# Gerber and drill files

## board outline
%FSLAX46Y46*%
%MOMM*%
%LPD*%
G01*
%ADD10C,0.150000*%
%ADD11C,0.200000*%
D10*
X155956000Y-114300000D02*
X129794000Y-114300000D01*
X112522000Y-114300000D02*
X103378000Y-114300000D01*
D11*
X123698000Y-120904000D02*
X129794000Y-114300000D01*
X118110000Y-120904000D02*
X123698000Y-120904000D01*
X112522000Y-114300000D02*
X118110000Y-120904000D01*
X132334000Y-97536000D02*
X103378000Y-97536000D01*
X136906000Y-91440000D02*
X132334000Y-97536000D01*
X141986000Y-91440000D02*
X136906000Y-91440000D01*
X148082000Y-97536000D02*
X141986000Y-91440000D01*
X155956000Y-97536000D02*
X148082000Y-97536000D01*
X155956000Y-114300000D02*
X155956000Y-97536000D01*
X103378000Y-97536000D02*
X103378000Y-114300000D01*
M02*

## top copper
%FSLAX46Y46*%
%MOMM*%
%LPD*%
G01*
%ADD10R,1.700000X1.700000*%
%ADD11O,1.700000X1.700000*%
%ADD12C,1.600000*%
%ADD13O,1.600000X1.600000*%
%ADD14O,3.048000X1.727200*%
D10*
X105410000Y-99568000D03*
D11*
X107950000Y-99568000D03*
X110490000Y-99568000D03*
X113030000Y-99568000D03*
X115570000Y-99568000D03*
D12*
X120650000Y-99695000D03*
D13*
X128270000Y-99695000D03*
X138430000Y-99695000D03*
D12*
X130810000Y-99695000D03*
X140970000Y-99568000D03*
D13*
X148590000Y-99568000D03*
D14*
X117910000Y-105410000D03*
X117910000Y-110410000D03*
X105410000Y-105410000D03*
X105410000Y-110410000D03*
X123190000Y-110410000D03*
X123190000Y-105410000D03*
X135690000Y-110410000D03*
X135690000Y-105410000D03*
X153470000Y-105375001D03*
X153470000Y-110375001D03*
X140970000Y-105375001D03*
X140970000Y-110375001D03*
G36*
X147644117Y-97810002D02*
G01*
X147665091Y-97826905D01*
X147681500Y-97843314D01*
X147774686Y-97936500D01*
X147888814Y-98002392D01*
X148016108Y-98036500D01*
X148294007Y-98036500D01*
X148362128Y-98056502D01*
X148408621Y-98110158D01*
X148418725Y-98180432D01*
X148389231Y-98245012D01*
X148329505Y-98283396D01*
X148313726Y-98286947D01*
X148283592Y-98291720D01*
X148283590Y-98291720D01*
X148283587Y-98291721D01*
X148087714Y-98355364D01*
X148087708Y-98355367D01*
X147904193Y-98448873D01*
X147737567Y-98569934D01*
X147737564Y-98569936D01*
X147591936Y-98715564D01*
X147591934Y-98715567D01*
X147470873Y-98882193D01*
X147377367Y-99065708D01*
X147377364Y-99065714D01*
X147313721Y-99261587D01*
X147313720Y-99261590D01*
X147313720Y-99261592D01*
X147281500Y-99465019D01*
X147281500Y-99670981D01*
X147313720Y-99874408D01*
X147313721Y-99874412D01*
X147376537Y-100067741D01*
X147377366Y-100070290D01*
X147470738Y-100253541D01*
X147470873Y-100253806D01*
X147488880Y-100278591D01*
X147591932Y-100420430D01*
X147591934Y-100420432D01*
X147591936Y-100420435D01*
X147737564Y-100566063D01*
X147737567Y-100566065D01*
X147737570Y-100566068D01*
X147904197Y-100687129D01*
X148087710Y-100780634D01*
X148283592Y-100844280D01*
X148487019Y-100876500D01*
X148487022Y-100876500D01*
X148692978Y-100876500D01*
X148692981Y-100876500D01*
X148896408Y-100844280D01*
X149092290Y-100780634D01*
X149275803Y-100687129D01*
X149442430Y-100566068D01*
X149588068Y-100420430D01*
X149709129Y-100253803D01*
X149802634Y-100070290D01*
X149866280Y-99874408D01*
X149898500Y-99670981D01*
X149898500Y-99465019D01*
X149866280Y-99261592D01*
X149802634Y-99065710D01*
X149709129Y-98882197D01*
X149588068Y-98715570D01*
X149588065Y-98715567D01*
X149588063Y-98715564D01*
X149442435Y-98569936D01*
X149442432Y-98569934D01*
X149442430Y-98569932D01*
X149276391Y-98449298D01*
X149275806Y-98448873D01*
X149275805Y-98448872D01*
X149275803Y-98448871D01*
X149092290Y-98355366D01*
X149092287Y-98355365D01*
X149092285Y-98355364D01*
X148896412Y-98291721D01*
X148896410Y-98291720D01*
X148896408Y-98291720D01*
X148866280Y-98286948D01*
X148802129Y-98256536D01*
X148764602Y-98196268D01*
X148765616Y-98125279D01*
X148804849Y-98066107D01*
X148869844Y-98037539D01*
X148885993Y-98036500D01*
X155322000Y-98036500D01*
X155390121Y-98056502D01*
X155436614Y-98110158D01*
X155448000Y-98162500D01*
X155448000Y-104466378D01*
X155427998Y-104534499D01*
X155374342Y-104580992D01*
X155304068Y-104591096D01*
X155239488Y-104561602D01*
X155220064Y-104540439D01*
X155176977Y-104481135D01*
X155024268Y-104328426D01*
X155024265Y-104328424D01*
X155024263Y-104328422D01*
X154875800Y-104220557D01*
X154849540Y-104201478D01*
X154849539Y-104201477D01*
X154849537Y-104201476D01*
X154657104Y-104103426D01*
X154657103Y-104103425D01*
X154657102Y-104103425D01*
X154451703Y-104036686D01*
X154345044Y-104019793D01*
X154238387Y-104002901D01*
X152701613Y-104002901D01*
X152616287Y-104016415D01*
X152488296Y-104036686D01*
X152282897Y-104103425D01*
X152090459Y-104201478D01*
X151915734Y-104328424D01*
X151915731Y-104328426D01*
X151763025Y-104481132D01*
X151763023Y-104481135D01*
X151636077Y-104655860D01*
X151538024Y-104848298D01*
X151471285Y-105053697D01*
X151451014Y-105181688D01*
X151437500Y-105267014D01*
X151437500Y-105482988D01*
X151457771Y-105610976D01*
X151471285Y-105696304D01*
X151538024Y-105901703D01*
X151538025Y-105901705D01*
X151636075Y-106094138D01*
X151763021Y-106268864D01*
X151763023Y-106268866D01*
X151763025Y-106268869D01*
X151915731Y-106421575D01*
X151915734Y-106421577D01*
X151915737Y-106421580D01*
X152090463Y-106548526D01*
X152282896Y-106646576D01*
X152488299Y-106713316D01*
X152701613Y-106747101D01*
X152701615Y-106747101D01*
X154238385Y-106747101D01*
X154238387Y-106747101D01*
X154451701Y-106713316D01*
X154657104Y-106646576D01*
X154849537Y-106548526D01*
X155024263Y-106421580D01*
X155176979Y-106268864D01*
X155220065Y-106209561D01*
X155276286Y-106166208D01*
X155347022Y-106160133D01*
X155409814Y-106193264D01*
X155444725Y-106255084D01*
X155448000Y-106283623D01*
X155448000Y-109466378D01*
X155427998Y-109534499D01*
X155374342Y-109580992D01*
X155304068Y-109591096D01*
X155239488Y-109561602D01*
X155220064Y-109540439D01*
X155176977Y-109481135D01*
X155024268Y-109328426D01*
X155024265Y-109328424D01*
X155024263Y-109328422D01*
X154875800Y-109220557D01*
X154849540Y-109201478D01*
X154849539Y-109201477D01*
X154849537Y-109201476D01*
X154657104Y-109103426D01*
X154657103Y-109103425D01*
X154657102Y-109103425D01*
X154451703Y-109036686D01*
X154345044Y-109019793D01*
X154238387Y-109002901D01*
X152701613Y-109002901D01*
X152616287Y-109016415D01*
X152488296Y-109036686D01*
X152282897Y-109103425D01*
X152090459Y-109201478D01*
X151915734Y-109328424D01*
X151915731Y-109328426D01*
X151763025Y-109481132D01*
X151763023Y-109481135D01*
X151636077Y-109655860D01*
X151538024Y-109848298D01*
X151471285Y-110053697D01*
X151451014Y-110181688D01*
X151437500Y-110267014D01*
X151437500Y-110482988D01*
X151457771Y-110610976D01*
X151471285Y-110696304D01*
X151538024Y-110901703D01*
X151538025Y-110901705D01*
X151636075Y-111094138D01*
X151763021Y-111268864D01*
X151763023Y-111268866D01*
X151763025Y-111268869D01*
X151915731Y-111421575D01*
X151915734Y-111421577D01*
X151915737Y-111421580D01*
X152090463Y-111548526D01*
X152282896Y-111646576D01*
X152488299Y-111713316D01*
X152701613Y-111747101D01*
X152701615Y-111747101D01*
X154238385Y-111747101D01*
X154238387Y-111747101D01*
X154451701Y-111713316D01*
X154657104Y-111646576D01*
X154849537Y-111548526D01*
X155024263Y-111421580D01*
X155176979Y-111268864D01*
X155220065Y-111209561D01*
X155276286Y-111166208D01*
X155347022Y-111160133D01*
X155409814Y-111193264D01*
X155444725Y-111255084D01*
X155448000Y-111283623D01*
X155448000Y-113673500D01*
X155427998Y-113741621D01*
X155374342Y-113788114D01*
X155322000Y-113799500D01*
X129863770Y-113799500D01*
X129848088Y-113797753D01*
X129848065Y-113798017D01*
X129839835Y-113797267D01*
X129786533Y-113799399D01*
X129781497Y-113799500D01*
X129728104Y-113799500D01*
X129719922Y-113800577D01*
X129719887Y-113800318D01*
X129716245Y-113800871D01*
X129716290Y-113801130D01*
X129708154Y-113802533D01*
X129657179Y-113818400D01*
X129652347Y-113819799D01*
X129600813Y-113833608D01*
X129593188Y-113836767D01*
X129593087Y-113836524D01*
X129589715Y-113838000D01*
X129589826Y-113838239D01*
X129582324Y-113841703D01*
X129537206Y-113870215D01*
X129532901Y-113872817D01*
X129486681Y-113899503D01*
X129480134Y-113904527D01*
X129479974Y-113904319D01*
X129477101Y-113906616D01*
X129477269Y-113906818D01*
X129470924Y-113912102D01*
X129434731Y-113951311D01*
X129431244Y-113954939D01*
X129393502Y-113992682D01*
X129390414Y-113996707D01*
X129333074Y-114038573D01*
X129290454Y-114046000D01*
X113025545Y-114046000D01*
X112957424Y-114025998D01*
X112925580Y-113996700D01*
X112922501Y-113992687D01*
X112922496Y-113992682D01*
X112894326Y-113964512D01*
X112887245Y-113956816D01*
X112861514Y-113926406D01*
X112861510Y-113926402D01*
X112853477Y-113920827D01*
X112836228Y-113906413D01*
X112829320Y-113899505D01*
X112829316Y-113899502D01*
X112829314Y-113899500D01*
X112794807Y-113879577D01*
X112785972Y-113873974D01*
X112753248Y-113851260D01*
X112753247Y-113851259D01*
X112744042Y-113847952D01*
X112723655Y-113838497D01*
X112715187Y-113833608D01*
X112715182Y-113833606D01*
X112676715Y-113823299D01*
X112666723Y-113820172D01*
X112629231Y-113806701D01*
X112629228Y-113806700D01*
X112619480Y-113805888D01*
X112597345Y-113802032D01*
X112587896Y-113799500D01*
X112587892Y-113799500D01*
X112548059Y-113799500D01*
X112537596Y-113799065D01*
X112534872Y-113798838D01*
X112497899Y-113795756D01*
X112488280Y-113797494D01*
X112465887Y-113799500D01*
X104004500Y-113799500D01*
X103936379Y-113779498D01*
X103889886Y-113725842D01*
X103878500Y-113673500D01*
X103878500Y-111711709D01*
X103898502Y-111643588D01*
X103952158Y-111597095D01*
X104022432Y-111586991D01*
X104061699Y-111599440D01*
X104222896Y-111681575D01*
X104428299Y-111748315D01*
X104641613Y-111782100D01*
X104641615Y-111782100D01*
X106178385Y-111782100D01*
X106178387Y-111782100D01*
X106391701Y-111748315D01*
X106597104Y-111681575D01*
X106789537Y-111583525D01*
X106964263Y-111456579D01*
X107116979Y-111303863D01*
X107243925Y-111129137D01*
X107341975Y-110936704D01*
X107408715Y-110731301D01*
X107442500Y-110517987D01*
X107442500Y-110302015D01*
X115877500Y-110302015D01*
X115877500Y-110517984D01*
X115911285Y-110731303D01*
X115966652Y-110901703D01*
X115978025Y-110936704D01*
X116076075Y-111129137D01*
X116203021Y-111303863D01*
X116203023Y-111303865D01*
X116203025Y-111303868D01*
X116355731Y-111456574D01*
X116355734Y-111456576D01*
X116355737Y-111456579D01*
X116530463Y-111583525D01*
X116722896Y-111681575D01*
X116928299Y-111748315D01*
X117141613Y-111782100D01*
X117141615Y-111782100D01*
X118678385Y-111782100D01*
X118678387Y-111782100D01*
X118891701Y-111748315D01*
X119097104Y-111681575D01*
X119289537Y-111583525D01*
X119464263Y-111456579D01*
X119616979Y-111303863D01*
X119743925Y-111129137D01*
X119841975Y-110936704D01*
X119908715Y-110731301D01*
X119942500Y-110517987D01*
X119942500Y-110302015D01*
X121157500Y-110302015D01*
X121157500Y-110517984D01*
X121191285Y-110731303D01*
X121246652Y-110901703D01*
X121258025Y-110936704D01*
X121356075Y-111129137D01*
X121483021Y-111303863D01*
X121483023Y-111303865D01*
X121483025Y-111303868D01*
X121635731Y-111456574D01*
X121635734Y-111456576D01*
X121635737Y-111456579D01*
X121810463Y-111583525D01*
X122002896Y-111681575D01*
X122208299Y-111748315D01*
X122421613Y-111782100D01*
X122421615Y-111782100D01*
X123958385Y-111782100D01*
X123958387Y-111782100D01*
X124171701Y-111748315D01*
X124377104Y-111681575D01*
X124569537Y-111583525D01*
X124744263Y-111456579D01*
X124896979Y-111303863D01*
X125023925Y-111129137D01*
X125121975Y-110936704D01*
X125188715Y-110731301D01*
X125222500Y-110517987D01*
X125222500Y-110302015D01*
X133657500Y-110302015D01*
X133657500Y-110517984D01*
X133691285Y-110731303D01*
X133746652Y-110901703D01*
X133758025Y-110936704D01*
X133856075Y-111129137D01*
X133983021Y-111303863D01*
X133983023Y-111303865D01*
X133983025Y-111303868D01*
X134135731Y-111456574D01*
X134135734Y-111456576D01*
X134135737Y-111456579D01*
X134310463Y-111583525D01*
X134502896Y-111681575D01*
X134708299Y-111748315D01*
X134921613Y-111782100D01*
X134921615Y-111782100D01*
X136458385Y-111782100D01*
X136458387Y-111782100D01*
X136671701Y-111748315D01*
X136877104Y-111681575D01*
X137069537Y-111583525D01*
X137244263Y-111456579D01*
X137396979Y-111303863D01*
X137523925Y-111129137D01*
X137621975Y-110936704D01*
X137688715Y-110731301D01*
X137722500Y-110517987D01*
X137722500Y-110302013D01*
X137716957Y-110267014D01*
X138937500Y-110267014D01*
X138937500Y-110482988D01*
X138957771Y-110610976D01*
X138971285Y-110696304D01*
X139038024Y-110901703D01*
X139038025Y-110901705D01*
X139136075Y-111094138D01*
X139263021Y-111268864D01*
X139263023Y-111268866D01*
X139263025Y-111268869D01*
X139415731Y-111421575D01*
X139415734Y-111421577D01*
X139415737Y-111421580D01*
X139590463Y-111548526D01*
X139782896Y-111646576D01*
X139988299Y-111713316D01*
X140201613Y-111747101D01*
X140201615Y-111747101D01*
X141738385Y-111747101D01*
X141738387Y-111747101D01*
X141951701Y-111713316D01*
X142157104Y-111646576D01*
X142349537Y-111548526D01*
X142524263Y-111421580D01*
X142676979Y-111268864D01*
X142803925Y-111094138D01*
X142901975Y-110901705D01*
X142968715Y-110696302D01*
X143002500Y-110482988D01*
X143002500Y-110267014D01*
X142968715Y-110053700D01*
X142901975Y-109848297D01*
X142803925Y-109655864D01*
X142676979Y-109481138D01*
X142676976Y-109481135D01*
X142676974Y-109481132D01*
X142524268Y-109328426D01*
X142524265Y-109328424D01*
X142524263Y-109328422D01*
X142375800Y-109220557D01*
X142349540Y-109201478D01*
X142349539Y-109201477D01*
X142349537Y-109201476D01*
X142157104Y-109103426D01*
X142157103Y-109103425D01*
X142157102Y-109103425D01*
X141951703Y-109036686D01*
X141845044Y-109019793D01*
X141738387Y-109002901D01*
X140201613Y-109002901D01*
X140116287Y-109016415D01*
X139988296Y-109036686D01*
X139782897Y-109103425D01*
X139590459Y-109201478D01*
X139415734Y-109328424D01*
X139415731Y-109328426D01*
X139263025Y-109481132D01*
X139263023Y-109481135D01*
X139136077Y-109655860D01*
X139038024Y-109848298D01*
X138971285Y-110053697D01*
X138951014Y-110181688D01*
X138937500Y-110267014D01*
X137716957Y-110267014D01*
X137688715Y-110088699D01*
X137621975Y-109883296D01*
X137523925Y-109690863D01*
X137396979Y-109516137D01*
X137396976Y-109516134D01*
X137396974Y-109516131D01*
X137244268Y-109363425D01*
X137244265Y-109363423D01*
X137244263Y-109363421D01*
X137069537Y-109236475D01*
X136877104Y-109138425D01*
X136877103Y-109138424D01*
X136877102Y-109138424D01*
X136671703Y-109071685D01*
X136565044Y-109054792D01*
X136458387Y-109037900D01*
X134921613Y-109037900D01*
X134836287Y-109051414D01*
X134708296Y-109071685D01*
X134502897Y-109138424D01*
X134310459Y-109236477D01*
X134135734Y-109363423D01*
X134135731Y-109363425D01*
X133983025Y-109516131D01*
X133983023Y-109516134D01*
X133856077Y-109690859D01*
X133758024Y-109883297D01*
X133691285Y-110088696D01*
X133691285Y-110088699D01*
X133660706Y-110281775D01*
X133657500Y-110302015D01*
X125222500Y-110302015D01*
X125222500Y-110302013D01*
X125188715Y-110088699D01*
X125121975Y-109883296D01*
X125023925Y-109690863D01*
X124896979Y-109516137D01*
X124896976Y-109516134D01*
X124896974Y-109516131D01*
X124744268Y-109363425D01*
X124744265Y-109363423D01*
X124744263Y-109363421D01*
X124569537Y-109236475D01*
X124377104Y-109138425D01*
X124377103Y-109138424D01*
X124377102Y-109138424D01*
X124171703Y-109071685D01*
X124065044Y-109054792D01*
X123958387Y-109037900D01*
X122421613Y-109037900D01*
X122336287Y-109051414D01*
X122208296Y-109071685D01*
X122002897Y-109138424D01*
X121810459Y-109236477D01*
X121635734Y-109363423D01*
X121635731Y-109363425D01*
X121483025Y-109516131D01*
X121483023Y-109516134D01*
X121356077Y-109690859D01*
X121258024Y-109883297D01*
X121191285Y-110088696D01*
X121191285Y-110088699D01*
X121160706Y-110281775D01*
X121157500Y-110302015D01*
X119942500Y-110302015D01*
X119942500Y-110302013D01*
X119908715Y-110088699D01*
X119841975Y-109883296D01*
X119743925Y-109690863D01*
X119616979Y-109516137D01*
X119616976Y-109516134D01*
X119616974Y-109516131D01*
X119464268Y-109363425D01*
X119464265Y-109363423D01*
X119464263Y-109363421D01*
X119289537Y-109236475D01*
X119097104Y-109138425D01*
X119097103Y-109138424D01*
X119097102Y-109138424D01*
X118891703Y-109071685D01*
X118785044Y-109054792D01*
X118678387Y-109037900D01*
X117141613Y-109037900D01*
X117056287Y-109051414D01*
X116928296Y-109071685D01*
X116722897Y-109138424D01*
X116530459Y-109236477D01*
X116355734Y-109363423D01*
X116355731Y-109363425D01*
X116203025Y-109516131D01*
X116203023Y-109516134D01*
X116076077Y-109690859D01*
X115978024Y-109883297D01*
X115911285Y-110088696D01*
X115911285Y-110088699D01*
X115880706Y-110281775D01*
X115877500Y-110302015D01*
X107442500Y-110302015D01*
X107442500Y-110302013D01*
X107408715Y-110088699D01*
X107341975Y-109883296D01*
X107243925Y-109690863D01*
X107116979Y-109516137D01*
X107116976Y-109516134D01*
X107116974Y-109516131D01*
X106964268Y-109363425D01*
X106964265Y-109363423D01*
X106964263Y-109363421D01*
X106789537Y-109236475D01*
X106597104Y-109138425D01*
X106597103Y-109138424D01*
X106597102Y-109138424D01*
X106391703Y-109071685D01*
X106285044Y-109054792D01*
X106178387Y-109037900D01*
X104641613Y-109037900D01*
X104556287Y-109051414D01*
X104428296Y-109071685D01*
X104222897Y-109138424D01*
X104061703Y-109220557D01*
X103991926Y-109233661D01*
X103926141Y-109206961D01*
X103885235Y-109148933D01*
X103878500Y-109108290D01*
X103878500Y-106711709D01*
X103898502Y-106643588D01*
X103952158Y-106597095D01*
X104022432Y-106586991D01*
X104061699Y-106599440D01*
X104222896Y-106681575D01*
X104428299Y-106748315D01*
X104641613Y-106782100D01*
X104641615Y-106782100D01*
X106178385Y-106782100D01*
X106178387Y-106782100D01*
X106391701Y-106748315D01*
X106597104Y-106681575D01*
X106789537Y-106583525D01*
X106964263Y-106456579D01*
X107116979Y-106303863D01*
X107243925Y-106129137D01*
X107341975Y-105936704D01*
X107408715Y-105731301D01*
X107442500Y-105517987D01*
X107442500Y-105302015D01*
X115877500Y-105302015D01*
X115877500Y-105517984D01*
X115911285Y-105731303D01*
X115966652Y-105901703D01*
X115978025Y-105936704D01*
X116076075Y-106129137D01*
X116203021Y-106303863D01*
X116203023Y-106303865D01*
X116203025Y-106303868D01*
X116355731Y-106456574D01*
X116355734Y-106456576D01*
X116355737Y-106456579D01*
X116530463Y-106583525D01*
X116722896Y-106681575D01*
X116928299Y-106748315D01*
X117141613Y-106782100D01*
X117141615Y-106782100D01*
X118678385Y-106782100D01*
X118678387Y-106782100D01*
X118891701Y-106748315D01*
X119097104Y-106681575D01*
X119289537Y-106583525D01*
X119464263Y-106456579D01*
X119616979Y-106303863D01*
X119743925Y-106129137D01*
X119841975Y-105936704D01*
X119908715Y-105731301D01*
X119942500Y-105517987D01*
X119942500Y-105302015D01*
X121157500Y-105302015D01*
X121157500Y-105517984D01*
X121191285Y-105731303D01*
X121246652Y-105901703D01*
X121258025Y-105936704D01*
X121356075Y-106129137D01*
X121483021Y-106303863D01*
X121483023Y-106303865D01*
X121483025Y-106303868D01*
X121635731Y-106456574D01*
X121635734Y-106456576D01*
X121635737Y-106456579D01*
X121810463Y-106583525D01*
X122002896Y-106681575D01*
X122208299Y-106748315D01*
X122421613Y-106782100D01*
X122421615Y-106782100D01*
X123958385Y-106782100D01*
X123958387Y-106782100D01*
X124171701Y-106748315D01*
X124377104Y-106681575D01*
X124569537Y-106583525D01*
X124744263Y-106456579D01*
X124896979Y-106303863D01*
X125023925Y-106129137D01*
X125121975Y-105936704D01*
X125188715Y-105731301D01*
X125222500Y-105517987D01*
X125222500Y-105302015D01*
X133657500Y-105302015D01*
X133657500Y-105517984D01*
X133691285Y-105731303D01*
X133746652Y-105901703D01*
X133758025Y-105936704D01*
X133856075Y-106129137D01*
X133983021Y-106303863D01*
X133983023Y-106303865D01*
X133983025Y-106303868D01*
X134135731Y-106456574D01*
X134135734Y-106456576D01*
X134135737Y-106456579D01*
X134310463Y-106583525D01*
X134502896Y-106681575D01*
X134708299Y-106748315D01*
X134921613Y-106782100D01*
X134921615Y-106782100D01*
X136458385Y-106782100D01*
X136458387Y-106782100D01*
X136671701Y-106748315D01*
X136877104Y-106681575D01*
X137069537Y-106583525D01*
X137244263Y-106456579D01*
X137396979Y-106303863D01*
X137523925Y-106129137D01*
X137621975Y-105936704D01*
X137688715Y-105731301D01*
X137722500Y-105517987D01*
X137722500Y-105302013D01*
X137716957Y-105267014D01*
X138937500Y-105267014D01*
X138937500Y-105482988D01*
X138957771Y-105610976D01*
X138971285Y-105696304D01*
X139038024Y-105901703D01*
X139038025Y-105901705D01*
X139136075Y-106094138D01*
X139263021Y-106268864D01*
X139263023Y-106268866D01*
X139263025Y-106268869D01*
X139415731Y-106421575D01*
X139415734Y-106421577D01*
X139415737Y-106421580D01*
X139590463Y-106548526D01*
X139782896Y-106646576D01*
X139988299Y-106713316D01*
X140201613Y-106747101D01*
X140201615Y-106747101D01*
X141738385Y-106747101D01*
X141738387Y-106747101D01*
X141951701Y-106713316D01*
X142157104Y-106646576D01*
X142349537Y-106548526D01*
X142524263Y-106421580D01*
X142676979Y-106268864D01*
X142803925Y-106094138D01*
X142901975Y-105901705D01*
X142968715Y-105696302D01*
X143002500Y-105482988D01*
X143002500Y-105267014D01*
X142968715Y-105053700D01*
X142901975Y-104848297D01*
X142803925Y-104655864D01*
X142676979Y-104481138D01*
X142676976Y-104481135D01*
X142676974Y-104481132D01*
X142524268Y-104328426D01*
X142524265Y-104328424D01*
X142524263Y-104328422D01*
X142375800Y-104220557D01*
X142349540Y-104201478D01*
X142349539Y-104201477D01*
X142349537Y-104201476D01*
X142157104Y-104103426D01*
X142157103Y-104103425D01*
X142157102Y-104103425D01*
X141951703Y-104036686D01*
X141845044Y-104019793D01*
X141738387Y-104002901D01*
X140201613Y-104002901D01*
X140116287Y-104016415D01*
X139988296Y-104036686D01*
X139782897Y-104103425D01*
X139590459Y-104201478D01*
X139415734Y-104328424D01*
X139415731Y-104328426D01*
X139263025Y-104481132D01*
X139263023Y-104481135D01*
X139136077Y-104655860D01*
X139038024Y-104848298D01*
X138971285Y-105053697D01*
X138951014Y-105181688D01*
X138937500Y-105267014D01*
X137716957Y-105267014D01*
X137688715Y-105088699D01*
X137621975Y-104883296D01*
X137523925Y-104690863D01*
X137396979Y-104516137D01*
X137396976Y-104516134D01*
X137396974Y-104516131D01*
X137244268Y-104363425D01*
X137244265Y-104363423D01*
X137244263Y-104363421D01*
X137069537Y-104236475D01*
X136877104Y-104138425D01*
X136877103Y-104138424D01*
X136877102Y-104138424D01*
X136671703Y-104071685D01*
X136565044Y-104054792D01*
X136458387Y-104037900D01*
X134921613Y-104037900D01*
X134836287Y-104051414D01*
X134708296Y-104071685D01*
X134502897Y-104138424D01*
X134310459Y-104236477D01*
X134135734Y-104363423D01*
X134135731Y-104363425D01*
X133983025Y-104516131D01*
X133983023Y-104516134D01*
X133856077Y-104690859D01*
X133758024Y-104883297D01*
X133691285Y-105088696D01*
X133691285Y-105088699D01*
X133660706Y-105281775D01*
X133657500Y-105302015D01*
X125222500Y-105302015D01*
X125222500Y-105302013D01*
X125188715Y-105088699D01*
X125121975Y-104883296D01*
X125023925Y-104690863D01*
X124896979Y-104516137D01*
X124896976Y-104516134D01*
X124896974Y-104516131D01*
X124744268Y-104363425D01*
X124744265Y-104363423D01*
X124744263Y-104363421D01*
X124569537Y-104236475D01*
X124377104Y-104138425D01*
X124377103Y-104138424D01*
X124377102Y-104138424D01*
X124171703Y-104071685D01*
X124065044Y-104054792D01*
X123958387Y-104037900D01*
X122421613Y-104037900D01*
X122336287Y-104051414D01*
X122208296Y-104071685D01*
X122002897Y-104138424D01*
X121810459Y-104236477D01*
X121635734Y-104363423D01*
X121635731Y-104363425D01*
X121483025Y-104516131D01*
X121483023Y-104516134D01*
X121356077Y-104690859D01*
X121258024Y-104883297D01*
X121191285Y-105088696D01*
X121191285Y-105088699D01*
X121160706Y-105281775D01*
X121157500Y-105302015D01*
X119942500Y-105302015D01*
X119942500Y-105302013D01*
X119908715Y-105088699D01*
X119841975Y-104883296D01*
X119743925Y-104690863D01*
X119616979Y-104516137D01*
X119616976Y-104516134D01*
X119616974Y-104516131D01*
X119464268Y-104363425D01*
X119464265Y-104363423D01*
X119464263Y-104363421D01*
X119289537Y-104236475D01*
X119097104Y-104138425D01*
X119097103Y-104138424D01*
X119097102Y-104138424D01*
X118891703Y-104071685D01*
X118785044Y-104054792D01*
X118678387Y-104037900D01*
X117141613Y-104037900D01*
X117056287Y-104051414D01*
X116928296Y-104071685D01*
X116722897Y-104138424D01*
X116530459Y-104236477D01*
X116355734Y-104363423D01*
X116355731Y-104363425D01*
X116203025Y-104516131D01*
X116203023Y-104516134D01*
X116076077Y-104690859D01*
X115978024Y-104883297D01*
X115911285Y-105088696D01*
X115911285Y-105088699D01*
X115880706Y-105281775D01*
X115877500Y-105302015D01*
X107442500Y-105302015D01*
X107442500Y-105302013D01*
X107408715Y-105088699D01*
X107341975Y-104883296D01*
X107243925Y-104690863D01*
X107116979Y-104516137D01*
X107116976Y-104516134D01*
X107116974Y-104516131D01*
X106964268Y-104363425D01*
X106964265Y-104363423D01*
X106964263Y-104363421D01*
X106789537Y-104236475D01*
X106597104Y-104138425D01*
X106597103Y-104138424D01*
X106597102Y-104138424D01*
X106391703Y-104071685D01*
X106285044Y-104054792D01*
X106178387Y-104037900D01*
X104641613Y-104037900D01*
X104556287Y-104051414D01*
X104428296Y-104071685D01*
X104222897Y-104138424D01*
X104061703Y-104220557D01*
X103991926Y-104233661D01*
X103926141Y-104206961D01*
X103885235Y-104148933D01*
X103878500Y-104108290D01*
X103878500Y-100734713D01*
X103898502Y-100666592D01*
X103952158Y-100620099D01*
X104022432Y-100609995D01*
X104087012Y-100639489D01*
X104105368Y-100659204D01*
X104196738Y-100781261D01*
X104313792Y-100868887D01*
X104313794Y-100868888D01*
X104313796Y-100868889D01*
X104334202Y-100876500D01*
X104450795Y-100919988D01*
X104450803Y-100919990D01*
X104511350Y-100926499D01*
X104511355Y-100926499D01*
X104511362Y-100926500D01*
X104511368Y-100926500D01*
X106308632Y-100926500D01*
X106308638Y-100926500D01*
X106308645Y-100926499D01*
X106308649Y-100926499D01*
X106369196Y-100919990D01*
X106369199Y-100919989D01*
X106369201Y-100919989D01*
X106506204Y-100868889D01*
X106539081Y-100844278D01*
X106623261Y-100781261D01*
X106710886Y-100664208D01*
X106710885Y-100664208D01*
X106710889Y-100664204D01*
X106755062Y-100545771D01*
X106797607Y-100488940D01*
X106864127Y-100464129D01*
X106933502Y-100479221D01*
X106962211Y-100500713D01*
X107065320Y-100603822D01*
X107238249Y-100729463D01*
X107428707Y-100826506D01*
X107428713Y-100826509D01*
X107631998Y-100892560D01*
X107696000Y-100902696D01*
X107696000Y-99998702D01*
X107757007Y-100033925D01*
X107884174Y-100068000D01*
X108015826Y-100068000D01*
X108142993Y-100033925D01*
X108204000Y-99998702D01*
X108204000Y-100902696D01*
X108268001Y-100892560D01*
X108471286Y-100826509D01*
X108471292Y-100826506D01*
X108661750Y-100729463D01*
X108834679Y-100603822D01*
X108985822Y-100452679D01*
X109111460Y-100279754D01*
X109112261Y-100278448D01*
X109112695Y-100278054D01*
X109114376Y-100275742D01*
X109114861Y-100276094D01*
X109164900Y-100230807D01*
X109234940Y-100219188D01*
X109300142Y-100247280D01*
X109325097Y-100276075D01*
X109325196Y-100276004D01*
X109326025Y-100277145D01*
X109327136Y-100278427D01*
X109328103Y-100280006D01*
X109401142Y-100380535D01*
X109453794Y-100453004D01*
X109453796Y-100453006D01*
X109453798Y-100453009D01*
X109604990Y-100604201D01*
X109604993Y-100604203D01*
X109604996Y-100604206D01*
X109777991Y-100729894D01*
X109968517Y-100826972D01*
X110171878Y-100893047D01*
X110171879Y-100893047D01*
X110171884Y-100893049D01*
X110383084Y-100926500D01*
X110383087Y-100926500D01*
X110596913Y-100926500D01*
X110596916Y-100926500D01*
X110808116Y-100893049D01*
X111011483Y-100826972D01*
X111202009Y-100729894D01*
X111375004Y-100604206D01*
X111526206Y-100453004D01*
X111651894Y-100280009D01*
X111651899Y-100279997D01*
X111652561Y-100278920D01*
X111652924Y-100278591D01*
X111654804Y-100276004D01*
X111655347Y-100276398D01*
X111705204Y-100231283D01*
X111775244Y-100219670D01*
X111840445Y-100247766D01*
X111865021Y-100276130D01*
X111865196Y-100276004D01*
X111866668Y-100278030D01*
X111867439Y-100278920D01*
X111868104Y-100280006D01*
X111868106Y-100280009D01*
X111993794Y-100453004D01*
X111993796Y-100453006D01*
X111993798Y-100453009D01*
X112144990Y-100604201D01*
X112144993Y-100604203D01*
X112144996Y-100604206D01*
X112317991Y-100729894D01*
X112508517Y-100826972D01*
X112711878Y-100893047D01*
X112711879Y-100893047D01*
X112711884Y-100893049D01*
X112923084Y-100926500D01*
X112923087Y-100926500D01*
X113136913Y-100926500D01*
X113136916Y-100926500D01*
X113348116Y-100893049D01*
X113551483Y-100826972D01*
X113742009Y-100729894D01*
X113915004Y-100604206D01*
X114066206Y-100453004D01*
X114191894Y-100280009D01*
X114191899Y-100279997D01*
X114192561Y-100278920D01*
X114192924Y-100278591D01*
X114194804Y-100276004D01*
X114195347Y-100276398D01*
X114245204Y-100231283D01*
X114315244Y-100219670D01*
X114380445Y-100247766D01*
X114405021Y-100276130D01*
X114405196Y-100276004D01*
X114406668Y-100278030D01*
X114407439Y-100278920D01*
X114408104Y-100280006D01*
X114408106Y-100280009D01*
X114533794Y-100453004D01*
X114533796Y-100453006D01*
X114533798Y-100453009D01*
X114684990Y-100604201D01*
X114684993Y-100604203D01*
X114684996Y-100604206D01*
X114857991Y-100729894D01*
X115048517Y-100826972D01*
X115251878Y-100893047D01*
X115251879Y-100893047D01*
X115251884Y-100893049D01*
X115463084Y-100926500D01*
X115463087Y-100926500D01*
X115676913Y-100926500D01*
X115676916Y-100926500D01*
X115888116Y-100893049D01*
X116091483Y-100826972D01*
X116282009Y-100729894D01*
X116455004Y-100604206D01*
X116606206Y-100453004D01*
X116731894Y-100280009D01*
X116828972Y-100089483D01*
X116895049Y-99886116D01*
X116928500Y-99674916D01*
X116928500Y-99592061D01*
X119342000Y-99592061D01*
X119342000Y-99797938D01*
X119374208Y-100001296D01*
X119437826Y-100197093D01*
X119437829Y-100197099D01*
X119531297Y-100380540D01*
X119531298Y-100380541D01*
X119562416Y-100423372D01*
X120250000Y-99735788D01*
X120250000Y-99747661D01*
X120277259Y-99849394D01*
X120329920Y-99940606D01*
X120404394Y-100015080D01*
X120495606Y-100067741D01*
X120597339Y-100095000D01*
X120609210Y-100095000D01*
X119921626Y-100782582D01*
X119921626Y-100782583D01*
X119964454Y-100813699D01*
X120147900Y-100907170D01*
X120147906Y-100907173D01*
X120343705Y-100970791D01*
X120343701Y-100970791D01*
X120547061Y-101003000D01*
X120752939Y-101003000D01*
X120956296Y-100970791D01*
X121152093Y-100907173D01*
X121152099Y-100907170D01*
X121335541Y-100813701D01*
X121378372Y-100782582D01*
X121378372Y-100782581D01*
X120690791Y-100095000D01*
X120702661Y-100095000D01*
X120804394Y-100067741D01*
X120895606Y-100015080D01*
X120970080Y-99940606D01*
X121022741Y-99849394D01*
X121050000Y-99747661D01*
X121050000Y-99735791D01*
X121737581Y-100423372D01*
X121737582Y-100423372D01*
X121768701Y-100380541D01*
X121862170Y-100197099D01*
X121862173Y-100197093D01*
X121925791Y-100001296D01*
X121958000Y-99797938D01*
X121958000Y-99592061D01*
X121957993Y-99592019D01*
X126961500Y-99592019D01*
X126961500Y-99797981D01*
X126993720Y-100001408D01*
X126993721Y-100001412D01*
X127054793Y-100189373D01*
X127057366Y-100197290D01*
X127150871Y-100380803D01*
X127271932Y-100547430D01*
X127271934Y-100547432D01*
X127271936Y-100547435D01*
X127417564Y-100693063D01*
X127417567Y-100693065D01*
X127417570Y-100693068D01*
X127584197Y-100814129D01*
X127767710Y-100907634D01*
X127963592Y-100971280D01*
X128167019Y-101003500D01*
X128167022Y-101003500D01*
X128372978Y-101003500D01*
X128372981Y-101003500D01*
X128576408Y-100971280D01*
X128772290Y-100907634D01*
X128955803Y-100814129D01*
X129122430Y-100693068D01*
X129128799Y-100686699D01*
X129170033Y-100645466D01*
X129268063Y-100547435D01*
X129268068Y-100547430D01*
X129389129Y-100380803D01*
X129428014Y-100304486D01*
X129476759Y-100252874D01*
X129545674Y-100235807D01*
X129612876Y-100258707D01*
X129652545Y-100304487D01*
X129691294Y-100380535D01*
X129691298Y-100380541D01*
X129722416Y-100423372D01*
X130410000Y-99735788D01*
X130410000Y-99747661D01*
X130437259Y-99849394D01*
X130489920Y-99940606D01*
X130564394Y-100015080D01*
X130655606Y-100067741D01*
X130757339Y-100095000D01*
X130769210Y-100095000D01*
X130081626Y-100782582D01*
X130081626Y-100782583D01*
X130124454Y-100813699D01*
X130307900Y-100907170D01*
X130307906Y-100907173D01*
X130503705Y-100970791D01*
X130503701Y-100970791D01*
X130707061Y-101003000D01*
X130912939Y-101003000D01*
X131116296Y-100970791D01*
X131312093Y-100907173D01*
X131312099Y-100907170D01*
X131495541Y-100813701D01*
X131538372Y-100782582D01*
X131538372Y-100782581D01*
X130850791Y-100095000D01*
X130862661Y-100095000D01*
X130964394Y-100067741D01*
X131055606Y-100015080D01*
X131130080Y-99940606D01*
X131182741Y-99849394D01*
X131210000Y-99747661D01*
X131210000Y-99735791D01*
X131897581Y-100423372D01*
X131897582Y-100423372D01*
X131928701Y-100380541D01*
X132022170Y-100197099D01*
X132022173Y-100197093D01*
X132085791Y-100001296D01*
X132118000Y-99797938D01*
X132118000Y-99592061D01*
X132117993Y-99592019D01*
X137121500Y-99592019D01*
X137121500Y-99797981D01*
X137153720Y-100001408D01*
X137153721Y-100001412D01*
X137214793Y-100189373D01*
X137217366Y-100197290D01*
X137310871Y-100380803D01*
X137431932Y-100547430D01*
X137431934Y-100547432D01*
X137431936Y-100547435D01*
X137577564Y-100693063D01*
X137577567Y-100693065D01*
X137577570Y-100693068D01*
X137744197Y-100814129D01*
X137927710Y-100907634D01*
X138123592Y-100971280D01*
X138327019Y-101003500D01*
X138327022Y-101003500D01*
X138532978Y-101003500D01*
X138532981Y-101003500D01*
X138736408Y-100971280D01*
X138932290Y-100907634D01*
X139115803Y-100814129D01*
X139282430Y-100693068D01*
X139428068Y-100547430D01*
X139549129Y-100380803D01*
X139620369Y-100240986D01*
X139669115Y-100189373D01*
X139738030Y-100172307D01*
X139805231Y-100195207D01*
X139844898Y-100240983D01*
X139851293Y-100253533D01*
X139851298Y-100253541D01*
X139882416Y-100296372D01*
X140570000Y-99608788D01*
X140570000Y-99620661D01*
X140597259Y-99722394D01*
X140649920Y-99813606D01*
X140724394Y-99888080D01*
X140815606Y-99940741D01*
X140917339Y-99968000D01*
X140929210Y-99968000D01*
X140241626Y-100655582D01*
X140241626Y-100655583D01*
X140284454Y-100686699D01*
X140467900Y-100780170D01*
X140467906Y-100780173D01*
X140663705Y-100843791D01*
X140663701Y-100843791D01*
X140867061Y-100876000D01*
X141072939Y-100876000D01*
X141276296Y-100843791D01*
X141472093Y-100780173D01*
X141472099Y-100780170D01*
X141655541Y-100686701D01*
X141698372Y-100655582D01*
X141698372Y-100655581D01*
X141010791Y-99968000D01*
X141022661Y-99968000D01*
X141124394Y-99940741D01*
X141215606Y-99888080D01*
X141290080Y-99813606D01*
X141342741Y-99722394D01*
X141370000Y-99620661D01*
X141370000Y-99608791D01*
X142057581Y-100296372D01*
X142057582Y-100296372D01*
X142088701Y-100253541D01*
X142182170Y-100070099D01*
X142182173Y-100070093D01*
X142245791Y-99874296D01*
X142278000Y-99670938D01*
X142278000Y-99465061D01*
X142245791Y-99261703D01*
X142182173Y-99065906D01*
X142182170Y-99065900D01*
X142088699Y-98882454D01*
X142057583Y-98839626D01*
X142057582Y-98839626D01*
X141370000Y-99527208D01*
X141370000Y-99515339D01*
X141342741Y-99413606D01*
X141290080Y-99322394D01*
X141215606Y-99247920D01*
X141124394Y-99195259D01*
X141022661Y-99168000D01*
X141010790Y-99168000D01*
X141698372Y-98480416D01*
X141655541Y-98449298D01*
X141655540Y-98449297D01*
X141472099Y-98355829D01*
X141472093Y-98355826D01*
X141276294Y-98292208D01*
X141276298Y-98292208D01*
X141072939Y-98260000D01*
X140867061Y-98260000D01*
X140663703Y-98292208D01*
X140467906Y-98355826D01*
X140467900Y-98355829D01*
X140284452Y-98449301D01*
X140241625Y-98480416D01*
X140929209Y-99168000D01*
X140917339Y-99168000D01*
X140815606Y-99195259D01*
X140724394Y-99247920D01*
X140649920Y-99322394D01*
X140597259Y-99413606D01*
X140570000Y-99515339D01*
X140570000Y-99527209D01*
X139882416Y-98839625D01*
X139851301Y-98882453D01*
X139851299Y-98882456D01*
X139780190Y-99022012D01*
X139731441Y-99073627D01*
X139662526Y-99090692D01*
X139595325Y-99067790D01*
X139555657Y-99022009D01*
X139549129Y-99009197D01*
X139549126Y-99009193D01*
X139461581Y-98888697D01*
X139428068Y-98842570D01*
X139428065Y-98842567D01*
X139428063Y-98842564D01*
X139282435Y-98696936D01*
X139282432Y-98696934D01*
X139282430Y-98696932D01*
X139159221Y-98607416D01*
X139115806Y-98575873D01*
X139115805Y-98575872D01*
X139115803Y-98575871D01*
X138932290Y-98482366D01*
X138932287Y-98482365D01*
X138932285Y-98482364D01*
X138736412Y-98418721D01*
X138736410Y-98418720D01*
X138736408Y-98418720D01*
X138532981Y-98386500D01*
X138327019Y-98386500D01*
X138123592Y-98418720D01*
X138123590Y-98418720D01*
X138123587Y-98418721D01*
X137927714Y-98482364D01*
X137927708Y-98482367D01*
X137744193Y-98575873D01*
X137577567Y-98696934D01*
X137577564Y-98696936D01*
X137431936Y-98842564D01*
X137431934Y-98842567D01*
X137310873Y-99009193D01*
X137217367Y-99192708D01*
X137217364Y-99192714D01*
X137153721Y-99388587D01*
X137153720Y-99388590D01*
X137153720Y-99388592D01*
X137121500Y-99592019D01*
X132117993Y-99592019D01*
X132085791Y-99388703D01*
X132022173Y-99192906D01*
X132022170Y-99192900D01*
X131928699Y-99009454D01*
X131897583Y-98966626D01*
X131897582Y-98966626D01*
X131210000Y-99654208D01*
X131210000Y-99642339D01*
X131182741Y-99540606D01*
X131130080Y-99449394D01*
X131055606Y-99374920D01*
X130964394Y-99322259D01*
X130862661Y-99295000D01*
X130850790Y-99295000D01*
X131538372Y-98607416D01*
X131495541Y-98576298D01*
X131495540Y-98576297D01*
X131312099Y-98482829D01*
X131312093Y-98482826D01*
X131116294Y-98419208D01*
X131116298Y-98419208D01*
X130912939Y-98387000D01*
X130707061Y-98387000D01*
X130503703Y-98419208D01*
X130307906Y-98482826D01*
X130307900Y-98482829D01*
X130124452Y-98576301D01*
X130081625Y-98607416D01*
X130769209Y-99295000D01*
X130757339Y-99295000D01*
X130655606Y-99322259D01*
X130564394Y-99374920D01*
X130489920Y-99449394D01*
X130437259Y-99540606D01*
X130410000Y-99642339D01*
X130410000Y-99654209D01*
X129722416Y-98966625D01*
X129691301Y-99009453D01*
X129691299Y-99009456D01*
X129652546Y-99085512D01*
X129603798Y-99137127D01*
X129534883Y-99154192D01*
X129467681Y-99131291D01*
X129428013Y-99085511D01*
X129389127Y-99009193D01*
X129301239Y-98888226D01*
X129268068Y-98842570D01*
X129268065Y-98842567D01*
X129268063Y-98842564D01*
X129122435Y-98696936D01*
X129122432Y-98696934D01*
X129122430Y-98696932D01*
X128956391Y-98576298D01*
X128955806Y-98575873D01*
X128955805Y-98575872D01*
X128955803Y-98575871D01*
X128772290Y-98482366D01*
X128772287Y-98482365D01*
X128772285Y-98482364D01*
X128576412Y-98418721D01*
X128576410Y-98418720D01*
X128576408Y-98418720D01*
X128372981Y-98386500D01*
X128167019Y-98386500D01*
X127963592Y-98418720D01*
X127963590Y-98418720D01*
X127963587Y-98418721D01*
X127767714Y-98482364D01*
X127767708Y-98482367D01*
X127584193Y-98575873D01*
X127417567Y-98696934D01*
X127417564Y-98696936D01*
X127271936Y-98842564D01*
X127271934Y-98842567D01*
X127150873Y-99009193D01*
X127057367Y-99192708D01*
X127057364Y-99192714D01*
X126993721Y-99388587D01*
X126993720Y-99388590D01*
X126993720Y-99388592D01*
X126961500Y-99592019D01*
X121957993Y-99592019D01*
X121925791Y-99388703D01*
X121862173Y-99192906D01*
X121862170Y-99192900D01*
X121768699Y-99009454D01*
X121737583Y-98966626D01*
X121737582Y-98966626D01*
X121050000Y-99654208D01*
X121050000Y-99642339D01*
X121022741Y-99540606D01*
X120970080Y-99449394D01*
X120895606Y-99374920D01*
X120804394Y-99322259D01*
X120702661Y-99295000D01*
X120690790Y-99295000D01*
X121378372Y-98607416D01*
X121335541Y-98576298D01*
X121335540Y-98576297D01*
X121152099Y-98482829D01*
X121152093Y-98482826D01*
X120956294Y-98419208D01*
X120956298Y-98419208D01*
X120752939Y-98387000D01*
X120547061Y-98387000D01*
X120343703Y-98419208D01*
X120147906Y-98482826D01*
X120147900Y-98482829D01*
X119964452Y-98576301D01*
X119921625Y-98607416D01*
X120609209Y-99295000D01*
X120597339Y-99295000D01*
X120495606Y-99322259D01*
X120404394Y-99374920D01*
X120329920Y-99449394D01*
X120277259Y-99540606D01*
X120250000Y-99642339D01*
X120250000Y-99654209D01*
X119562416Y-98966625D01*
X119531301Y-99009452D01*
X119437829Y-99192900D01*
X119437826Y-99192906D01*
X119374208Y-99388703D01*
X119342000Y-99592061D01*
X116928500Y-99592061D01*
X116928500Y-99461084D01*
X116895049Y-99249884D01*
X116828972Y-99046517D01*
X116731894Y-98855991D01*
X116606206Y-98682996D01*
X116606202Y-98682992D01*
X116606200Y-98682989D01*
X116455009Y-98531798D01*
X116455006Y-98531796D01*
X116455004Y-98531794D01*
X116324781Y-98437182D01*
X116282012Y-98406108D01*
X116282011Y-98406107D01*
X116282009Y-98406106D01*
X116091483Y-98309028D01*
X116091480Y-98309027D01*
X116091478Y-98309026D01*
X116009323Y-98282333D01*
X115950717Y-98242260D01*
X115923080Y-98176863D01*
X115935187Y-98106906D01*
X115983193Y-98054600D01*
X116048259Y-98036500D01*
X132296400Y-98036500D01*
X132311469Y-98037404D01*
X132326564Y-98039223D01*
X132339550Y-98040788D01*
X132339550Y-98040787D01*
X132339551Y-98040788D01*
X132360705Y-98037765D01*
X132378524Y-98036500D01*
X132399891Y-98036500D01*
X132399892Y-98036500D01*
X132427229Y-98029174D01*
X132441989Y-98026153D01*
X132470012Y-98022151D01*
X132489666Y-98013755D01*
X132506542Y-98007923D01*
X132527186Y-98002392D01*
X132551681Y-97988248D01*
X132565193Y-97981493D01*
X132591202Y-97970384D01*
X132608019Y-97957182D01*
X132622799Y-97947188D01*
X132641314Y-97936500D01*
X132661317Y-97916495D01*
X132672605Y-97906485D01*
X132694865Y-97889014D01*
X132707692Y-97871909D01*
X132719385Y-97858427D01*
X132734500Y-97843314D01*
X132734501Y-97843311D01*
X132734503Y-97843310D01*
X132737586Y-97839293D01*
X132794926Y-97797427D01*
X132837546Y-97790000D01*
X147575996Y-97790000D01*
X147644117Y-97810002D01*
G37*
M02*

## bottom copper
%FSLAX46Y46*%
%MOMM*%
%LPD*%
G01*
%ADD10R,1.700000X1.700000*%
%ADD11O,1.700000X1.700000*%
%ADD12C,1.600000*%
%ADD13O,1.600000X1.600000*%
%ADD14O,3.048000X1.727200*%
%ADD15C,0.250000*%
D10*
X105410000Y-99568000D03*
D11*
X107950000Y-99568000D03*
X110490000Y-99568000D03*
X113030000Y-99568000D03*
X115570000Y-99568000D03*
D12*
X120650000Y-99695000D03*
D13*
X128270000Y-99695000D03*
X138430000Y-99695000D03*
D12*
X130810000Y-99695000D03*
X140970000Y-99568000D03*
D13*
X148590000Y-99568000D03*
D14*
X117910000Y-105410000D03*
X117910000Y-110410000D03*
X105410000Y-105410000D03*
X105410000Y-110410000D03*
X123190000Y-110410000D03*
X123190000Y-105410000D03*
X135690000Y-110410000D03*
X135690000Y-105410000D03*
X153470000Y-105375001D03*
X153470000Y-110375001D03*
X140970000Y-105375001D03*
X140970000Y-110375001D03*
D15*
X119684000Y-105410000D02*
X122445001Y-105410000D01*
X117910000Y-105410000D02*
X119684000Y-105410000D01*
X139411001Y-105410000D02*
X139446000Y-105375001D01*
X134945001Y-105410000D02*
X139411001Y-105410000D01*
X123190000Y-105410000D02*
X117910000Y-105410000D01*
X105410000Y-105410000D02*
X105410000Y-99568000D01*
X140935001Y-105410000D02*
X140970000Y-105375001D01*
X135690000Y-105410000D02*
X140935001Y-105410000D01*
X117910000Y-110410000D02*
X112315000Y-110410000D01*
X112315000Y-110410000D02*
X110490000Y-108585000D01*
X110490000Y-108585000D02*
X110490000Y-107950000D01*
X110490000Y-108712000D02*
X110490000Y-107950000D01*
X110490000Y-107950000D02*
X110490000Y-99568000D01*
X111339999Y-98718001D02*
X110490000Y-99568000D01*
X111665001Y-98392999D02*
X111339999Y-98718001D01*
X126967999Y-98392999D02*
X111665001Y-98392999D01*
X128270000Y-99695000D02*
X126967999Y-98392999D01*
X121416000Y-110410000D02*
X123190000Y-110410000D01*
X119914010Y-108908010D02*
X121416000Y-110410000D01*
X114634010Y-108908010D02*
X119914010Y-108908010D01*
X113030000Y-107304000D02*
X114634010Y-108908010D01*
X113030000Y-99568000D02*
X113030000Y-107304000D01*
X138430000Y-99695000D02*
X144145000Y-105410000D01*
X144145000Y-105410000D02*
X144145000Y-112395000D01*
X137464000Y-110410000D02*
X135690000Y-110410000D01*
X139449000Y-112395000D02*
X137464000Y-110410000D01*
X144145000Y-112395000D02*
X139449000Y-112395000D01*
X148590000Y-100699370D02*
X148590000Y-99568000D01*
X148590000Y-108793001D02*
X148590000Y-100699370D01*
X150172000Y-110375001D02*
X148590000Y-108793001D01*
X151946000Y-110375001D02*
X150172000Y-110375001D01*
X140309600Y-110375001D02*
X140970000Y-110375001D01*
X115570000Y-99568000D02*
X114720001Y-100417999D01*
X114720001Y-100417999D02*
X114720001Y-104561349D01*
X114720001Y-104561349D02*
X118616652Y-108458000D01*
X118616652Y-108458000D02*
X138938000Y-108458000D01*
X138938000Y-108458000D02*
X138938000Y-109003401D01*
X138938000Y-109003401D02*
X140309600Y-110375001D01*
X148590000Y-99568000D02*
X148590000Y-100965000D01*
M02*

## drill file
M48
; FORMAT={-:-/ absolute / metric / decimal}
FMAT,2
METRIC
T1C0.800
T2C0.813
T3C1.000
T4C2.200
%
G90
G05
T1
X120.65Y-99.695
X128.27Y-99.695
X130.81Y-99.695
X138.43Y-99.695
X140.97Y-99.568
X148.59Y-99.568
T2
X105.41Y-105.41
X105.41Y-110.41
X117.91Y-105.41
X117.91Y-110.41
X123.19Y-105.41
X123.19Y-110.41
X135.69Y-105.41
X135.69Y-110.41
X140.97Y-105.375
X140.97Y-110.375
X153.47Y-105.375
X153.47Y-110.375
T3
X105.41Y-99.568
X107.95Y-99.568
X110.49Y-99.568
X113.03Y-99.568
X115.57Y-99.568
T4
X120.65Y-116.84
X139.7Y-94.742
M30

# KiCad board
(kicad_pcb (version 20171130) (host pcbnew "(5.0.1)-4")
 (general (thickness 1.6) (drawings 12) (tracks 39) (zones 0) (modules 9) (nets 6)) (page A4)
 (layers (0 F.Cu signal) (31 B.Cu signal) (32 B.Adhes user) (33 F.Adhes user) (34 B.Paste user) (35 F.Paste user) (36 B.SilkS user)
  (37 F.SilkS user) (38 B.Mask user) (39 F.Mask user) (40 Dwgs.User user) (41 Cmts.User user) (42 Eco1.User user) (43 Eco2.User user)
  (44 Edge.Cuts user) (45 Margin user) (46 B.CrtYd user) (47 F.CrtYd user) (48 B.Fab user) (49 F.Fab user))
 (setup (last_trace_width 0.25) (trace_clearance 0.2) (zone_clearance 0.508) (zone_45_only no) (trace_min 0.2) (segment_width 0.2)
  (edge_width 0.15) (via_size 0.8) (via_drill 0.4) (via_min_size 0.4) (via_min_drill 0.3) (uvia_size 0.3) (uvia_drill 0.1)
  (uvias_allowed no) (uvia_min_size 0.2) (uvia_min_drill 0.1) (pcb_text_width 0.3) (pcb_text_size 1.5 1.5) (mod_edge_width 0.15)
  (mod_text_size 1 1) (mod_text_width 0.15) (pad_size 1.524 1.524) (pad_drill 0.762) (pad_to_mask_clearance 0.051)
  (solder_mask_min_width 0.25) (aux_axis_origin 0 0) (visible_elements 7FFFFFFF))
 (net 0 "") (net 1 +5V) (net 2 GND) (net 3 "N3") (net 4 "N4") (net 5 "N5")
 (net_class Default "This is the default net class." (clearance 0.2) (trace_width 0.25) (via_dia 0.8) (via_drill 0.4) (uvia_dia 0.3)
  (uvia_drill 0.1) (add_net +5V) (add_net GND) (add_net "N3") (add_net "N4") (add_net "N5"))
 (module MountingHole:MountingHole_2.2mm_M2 (layer F.Cu) (at 139.7 94.742)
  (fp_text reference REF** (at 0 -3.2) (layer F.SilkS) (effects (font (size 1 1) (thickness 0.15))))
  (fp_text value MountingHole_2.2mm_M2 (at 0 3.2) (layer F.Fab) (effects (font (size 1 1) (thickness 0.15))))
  (pad 1 np_thru_hole circle (at 0 0) (size 2.2 2.2) (drill 2.2) (layers *.Cu *.Mask)))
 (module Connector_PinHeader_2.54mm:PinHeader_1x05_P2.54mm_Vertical (layer F.Cu) (at 105.41 99.568 90)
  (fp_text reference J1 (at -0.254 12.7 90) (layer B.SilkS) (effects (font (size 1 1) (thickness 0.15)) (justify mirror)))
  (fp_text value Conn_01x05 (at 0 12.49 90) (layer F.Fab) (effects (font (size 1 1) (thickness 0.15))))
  (pad 1 thru_hole rect (at 0 0 90) (size 1.7 1.7) (drill 1) (layers *.Cu *.Mask) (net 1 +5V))
  (pad 2 thru_hole oval (at 0 2.54 90) (size 1.7 1.7) (drill 1) (layers *.Cu *.Mask) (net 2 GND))
  (pad 3 thru_hole oval (at 0 5.08 90) (size 1.7 1.7) (drill 1) (layers *.Cu *.Mask) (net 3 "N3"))
  (pad 4 thru_hole oval (at 0 7.62 90) (size 1.7 1.7) (drill 1) (layers *.Cu *.Mask) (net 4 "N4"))
  (pad 5 thru_hole oval (at 0 10.16 90) (size 1.7 1.7) (drill 1) (layers *.Cu *.Mask) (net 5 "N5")))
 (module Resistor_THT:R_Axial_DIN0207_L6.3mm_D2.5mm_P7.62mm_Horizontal (layer F.Cu) (at 120.65 99.695)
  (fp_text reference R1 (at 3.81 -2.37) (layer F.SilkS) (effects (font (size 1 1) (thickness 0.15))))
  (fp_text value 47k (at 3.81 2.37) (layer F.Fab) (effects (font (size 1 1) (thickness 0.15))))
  (pad 1 thru_hole circle (at 0 0) (size 1.6 1.6) (drill 0.8) (layers *.Cu *.Mask) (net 2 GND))
  (pad 2 thru_hole oval (at 7.62 0) (size 1.6 1.6) (drill 0.8) (layers *.Cu *.Mask) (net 3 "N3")))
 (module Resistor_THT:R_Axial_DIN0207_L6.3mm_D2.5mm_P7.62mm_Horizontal (layer F.Cu) (at 130.81 99.695)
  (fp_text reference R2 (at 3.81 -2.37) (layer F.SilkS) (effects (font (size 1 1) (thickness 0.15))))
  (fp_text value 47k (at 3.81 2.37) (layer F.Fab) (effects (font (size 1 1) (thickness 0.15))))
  (pad 2 thru_hole oval (at 7.62 0) (size 1.6 1.6) (drill 0.8) (layers *.Cu *.Mask) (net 4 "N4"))
  (pad 1 thru_hole circle (at 0 0) (size 1.6 1.6) (drill 0.8) (layers *.Cu *.Mask) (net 2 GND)))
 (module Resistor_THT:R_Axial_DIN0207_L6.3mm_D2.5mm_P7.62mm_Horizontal (layer F.Cu) (at 140.97 99.568)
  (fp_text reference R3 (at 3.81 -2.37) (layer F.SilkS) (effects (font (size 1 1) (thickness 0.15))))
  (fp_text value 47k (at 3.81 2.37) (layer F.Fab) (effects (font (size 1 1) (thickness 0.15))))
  (pad 1 thru_hole circle (at 0 0) (size 1.6 1.6) (drill 0.8) (layers *.Cu *.Mask) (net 2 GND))
  (pad 2 thru_hole oval (at 7.62 0) (size 1.6 1.6) (drill 0.8) (layers *.Cu *.Mask) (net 5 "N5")))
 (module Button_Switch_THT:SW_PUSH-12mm (layer F.Cu) (at 105.41 105.41)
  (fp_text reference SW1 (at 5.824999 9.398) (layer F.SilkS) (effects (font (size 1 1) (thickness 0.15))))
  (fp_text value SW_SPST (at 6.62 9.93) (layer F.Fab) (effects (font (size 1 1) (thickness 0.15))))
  (pad 1 thru_hole oval (at 12.5 0) (size 3.048 1.7272) (drill 0.8128) (layers *.Cu *.Mask) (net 1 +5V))
  (pad 2 thru_hole oval (at 12.5 5) (size 3.048 1.7272) (drill 0.8128) (layers *.Cu *.Mask) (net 3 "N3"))
  (pad 1 thru_hole oval (at 0 0) (size 3.048 1.7272) (drill 0.8128) (layers *.Cu *.Mask) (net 1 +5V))
  (pad 2 thru_hole oval (at 0 5) (size 3.048 1.7272) (drill 0.8128) (layers *.Cu *.Mask) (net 3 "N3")))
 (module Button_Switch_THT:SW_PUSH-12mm (layer F.Cu) (at 123.19 105.41)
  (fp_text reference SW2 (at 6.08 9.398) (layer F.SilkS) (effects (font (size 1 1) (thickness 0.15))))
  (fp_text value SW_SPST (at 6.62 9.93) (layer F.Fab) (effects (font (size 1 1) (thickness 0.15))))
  (pad 2 thru_hole oval (at 0 5) (size 3.048 1.7272) (drill 0.8128) (layers *.Cu *.Mask) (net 4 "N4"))
  (pad 1 thru_hole oval (at 0 0) (size 3.048 1.7272) (drill 0.8128) (layers *.Cu *.Mask) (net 1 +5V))
  (pad 2 thru_hole oval (at 12.5 5) (size 3.048 1.7272) (drill 0.8128) (layers *.Cu *.Mask) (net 4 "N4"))
  (pad 1 thru_hole oval (at 12.5 0) (size 3.048 1.7272) (drill 0.8128) (layers *.Cu *.Mask) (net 1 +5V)))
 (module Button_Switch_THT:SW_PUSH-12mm (layer F.Cu) (at 140.97 105.375001)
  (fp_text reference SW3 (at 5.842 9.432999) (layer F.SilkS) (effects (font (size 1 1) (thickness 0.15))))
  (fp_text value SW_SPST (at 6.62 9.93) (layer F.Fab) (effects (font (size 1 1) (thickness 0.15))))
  (pad 1 thru_hole oval (at 12.5 0) (size 3.048 1.7272) (drill 0.8128) (layers *.Cu *.Mask) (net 1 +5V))
  (pad 2 thru_hole oval (at 12.5 5) (size 3.048 1.7272) (drill 0.8128) (layers *.Cu *.Mask) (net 5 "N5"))
  (pad 1 thru_hole oval (at 0 0) (size 3.048 1.7272) (drill 0.8128) (layers *.Cu *.Mask) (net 1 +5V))
  (pad 2 thru_hole oval (at 0 5) (size 3.048 1.7272) (drill 0.8128) (layers *.Cu *.Mask) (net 5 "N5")))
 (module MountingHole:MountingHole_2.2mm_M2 (layer F.Cu) (at 120.65 116.84)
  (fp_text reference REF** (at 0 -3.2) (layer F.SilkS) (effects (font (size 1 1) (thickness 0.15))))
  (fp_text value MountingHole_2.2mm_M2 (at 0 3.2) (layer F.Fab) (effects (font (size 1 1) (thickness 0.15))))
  (pad 1 np_thru_hole circle (at 0 0) (size 2.2 2.2) (drill 2.2) (layers *.Cu *.Mask)))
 (gr_line (start 155.956 114.3) (end 129.794 114.3) (layer Edge.Cuts) (width 0.15))
 (gr_line (start 112.522 114.3) (end 103.378 114.3) (layer Edge.Cuts) (width 0.15))
 (gr_line (start 123.698 120.904) (end 129.794 114.3) (layer Edge.Cuts) (width 0.2))
 (gr_line (start 118.11 120.904) (end 123.698 120.904) (layer Edge.Cuts) (width 0.2))
 (gr_line (start 112.522 114.3) (end 118.11 120.904) (layer Edge.Cuts) (width 0.2))
 (gr_line (start 132.334 97.536) (end 103.378 97.536) (layer Edge.Cuts) (width 0.2))
 (gr_line (start 136.906 91.44) (end 132.334 97.536) (layer Edge.Cuts) (width 0.2))
 (gr_line (start 141.986 91.44) (end 136.906 91.44) (layer Edge.Cuts) (width 0.2))
 (gr_line (start 148.082 97.536) (end 141.986 91.44) (layer Edge.Cuts) (width 0.2))
 (gr_line (start 155.956 97.536) (end 148.082 97.536) (layer Edge.Cuts) (width 0.2))
 (gr_line (start 155.956 114.3) (end 155.956 97.536) (layer Edge.Cuts) (width 0.2))
 (gr_line (start 103.378 97.536) (end 103.378 114.3) (layer Edge.Cuts) (width 0.2))
 (segment (start 119.684 105.41) (end 122.445001 105.41) (width 0.25) (layer B.Cu) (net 1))
 (segment (start 117.91 105.41) (end 119.684 105.41) (width 0.25) (layer B.Cu) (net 1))
 (segment (start 139.411001 105.41) (end 139.446 105.375001) (width 0.25) (layer B.Cu) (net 1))
 (segment (start 134.945001 105.41) (end 139.411001 105.41) (width 0.25) (layer B.Cu) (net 1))
 (segment (start 123.19 105.41) (end 117.91 105.41) (width 0.25) (layer B.Cu) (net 1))
 (segment (start 105.41 105.41) (end 105.41 99.568) (width 0.25) (layer B.Cu) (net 1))
 (segment (start 140.935001 105.41) (end 140.97 105.375001) (width 0.25) (layer B.Cu) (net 1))
 (segment (start 135.69 105.41) (end 140.935001 105.41) (width 0.25) (layer B.Cu) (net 1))
 (segment (start 117.91 110.41) (end 112.315 110.41) (width 0.25) (layer B.Cu) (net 3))
 (segment (start 112.315 110.41) (end 110.49 108.585) (width 0.25) (layer B.Cu) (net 3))
 (segment (start 110.49 108.585) (end 110.49 107.95) (width 0.25) (layer B.Cu) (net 3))
 (segment (start 110.49 108.712) (end 110.49 107.95) (width 0.25) (layer B.Cu) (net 3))
 (segment (start 110.49 107.95) (end 110.49 99.568) (width 0.25) (layer B.Cu) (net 3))
 (segment (start 111.339999 98.718001) (end 110.49 99.568) (width 0.25) (layer B.Cu) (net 3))
 (segment (start 111.665001 98.392999) (end 111.339999 98.718001) (width 0.25) (layer B.Cu) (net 3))
 (segment (start 126.967999 98.392999) (end 111.665001 98.392999) (width 0.25) (layer B.Cu) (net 3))
 (segment (start 128.27 99.695) (end 126.967999 98.392999) (width 0.25) (layer B.Cu) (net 3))
 (segment (start 121.416 110.41) (end 123.19 110.41) (width 0.25) (layer B.Cu) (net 4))
 (segment (start 119.91401 108.90801) (end 121.416 110.41) (width 0.25) (layer B.Cu) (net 4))
 (segment (start 114.63401 108.90801) (end 119.91401 108.90801) (width 0.25) (layer B.Cu) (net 4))
 (segment (start 113.03 107.304) (end 114.63401 108.90801) (width 0.25) (layer B.Cu) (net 4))
 (segment (start 113.03 99.568) (end 113.03 107.304) (width 0.25) (layer B.Cu) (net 4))
 (segment (start 138.43 99.695) (end 144.145 105.41) (width 0.25) (layer B.Cu) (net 4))
 (segment (start 144.145 105.41) (end 144.145 112.395) (width 0.25) (layer B.Cu) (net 4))
 (segment (start 137.464 110.41) (end 135.69 110.41) (width 0.25) (layer B.Cu) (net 4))
 (segment (start 139.449 112.395) (end 137.464 110.41) (width 0.25) (layer B.Cu) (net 4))
 (segment (start 144.145 112.395) (end 139.449 112.395) (width 0.25) (layer B.Cu) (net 4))
 (segment (start 148.59 100.69937) (end 148.59 99.568) (width 0.25) (layer B.Cu) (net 5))
 (segment (start 148.59 108.793001) (end 148.59 100.69937) (width 0.25) (layer B.Cu) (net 5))
 (segment (start 150.172 110.375001) (end 148.59 108.793001) (width 0.25) (layer B.Cu) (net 5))
 (segment (start 151.946 110.375001) (end 150.172 110.375001) (width 0.25) (layer B.Cu) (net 5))
 (segment (start 140.3096 110.375001) (end 140.97 110.375001) (width 0.25) (layer B.Cu) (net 5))
 (segment (start 115.57 99.568) (end 114.720001 100.417999) (width 0.25) (layer B.Cu) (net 5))
 (segment (start 114.720001 100.417999) (end 114.720001 104.561349) (width 0.25) (layer B.Cu) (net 5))
 (segment (start 114.720001 104.561349) (end 118.616652 108.458) (width 0.25) (layer B.Cu) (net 5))
 (segment (start 118.616652 108.458) (end 138.938 108.458) (width 0.25) (layer B.Cu) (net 5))
 (segment (start 138.938 108.458) (end 138.938 109.003401) (width 0.25) (layer B.Cu) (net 5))
 (segment (start 138.938 109.003401) (end 140.3096 110.375001) (width 0.25) (layer B.Cu) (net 5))
 (segment (start 148.59 99.568) (end 148.59 100.965) (width 0.25) (layer B.Cu) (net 5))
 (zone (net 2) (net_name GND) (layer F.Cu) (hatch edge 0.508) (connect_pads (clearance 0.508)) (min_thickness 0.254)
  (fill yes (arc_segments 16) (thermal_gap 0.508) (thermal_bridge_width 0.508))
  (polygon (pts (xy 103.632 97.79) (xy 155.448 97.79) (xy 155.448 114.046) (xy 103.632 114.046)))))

